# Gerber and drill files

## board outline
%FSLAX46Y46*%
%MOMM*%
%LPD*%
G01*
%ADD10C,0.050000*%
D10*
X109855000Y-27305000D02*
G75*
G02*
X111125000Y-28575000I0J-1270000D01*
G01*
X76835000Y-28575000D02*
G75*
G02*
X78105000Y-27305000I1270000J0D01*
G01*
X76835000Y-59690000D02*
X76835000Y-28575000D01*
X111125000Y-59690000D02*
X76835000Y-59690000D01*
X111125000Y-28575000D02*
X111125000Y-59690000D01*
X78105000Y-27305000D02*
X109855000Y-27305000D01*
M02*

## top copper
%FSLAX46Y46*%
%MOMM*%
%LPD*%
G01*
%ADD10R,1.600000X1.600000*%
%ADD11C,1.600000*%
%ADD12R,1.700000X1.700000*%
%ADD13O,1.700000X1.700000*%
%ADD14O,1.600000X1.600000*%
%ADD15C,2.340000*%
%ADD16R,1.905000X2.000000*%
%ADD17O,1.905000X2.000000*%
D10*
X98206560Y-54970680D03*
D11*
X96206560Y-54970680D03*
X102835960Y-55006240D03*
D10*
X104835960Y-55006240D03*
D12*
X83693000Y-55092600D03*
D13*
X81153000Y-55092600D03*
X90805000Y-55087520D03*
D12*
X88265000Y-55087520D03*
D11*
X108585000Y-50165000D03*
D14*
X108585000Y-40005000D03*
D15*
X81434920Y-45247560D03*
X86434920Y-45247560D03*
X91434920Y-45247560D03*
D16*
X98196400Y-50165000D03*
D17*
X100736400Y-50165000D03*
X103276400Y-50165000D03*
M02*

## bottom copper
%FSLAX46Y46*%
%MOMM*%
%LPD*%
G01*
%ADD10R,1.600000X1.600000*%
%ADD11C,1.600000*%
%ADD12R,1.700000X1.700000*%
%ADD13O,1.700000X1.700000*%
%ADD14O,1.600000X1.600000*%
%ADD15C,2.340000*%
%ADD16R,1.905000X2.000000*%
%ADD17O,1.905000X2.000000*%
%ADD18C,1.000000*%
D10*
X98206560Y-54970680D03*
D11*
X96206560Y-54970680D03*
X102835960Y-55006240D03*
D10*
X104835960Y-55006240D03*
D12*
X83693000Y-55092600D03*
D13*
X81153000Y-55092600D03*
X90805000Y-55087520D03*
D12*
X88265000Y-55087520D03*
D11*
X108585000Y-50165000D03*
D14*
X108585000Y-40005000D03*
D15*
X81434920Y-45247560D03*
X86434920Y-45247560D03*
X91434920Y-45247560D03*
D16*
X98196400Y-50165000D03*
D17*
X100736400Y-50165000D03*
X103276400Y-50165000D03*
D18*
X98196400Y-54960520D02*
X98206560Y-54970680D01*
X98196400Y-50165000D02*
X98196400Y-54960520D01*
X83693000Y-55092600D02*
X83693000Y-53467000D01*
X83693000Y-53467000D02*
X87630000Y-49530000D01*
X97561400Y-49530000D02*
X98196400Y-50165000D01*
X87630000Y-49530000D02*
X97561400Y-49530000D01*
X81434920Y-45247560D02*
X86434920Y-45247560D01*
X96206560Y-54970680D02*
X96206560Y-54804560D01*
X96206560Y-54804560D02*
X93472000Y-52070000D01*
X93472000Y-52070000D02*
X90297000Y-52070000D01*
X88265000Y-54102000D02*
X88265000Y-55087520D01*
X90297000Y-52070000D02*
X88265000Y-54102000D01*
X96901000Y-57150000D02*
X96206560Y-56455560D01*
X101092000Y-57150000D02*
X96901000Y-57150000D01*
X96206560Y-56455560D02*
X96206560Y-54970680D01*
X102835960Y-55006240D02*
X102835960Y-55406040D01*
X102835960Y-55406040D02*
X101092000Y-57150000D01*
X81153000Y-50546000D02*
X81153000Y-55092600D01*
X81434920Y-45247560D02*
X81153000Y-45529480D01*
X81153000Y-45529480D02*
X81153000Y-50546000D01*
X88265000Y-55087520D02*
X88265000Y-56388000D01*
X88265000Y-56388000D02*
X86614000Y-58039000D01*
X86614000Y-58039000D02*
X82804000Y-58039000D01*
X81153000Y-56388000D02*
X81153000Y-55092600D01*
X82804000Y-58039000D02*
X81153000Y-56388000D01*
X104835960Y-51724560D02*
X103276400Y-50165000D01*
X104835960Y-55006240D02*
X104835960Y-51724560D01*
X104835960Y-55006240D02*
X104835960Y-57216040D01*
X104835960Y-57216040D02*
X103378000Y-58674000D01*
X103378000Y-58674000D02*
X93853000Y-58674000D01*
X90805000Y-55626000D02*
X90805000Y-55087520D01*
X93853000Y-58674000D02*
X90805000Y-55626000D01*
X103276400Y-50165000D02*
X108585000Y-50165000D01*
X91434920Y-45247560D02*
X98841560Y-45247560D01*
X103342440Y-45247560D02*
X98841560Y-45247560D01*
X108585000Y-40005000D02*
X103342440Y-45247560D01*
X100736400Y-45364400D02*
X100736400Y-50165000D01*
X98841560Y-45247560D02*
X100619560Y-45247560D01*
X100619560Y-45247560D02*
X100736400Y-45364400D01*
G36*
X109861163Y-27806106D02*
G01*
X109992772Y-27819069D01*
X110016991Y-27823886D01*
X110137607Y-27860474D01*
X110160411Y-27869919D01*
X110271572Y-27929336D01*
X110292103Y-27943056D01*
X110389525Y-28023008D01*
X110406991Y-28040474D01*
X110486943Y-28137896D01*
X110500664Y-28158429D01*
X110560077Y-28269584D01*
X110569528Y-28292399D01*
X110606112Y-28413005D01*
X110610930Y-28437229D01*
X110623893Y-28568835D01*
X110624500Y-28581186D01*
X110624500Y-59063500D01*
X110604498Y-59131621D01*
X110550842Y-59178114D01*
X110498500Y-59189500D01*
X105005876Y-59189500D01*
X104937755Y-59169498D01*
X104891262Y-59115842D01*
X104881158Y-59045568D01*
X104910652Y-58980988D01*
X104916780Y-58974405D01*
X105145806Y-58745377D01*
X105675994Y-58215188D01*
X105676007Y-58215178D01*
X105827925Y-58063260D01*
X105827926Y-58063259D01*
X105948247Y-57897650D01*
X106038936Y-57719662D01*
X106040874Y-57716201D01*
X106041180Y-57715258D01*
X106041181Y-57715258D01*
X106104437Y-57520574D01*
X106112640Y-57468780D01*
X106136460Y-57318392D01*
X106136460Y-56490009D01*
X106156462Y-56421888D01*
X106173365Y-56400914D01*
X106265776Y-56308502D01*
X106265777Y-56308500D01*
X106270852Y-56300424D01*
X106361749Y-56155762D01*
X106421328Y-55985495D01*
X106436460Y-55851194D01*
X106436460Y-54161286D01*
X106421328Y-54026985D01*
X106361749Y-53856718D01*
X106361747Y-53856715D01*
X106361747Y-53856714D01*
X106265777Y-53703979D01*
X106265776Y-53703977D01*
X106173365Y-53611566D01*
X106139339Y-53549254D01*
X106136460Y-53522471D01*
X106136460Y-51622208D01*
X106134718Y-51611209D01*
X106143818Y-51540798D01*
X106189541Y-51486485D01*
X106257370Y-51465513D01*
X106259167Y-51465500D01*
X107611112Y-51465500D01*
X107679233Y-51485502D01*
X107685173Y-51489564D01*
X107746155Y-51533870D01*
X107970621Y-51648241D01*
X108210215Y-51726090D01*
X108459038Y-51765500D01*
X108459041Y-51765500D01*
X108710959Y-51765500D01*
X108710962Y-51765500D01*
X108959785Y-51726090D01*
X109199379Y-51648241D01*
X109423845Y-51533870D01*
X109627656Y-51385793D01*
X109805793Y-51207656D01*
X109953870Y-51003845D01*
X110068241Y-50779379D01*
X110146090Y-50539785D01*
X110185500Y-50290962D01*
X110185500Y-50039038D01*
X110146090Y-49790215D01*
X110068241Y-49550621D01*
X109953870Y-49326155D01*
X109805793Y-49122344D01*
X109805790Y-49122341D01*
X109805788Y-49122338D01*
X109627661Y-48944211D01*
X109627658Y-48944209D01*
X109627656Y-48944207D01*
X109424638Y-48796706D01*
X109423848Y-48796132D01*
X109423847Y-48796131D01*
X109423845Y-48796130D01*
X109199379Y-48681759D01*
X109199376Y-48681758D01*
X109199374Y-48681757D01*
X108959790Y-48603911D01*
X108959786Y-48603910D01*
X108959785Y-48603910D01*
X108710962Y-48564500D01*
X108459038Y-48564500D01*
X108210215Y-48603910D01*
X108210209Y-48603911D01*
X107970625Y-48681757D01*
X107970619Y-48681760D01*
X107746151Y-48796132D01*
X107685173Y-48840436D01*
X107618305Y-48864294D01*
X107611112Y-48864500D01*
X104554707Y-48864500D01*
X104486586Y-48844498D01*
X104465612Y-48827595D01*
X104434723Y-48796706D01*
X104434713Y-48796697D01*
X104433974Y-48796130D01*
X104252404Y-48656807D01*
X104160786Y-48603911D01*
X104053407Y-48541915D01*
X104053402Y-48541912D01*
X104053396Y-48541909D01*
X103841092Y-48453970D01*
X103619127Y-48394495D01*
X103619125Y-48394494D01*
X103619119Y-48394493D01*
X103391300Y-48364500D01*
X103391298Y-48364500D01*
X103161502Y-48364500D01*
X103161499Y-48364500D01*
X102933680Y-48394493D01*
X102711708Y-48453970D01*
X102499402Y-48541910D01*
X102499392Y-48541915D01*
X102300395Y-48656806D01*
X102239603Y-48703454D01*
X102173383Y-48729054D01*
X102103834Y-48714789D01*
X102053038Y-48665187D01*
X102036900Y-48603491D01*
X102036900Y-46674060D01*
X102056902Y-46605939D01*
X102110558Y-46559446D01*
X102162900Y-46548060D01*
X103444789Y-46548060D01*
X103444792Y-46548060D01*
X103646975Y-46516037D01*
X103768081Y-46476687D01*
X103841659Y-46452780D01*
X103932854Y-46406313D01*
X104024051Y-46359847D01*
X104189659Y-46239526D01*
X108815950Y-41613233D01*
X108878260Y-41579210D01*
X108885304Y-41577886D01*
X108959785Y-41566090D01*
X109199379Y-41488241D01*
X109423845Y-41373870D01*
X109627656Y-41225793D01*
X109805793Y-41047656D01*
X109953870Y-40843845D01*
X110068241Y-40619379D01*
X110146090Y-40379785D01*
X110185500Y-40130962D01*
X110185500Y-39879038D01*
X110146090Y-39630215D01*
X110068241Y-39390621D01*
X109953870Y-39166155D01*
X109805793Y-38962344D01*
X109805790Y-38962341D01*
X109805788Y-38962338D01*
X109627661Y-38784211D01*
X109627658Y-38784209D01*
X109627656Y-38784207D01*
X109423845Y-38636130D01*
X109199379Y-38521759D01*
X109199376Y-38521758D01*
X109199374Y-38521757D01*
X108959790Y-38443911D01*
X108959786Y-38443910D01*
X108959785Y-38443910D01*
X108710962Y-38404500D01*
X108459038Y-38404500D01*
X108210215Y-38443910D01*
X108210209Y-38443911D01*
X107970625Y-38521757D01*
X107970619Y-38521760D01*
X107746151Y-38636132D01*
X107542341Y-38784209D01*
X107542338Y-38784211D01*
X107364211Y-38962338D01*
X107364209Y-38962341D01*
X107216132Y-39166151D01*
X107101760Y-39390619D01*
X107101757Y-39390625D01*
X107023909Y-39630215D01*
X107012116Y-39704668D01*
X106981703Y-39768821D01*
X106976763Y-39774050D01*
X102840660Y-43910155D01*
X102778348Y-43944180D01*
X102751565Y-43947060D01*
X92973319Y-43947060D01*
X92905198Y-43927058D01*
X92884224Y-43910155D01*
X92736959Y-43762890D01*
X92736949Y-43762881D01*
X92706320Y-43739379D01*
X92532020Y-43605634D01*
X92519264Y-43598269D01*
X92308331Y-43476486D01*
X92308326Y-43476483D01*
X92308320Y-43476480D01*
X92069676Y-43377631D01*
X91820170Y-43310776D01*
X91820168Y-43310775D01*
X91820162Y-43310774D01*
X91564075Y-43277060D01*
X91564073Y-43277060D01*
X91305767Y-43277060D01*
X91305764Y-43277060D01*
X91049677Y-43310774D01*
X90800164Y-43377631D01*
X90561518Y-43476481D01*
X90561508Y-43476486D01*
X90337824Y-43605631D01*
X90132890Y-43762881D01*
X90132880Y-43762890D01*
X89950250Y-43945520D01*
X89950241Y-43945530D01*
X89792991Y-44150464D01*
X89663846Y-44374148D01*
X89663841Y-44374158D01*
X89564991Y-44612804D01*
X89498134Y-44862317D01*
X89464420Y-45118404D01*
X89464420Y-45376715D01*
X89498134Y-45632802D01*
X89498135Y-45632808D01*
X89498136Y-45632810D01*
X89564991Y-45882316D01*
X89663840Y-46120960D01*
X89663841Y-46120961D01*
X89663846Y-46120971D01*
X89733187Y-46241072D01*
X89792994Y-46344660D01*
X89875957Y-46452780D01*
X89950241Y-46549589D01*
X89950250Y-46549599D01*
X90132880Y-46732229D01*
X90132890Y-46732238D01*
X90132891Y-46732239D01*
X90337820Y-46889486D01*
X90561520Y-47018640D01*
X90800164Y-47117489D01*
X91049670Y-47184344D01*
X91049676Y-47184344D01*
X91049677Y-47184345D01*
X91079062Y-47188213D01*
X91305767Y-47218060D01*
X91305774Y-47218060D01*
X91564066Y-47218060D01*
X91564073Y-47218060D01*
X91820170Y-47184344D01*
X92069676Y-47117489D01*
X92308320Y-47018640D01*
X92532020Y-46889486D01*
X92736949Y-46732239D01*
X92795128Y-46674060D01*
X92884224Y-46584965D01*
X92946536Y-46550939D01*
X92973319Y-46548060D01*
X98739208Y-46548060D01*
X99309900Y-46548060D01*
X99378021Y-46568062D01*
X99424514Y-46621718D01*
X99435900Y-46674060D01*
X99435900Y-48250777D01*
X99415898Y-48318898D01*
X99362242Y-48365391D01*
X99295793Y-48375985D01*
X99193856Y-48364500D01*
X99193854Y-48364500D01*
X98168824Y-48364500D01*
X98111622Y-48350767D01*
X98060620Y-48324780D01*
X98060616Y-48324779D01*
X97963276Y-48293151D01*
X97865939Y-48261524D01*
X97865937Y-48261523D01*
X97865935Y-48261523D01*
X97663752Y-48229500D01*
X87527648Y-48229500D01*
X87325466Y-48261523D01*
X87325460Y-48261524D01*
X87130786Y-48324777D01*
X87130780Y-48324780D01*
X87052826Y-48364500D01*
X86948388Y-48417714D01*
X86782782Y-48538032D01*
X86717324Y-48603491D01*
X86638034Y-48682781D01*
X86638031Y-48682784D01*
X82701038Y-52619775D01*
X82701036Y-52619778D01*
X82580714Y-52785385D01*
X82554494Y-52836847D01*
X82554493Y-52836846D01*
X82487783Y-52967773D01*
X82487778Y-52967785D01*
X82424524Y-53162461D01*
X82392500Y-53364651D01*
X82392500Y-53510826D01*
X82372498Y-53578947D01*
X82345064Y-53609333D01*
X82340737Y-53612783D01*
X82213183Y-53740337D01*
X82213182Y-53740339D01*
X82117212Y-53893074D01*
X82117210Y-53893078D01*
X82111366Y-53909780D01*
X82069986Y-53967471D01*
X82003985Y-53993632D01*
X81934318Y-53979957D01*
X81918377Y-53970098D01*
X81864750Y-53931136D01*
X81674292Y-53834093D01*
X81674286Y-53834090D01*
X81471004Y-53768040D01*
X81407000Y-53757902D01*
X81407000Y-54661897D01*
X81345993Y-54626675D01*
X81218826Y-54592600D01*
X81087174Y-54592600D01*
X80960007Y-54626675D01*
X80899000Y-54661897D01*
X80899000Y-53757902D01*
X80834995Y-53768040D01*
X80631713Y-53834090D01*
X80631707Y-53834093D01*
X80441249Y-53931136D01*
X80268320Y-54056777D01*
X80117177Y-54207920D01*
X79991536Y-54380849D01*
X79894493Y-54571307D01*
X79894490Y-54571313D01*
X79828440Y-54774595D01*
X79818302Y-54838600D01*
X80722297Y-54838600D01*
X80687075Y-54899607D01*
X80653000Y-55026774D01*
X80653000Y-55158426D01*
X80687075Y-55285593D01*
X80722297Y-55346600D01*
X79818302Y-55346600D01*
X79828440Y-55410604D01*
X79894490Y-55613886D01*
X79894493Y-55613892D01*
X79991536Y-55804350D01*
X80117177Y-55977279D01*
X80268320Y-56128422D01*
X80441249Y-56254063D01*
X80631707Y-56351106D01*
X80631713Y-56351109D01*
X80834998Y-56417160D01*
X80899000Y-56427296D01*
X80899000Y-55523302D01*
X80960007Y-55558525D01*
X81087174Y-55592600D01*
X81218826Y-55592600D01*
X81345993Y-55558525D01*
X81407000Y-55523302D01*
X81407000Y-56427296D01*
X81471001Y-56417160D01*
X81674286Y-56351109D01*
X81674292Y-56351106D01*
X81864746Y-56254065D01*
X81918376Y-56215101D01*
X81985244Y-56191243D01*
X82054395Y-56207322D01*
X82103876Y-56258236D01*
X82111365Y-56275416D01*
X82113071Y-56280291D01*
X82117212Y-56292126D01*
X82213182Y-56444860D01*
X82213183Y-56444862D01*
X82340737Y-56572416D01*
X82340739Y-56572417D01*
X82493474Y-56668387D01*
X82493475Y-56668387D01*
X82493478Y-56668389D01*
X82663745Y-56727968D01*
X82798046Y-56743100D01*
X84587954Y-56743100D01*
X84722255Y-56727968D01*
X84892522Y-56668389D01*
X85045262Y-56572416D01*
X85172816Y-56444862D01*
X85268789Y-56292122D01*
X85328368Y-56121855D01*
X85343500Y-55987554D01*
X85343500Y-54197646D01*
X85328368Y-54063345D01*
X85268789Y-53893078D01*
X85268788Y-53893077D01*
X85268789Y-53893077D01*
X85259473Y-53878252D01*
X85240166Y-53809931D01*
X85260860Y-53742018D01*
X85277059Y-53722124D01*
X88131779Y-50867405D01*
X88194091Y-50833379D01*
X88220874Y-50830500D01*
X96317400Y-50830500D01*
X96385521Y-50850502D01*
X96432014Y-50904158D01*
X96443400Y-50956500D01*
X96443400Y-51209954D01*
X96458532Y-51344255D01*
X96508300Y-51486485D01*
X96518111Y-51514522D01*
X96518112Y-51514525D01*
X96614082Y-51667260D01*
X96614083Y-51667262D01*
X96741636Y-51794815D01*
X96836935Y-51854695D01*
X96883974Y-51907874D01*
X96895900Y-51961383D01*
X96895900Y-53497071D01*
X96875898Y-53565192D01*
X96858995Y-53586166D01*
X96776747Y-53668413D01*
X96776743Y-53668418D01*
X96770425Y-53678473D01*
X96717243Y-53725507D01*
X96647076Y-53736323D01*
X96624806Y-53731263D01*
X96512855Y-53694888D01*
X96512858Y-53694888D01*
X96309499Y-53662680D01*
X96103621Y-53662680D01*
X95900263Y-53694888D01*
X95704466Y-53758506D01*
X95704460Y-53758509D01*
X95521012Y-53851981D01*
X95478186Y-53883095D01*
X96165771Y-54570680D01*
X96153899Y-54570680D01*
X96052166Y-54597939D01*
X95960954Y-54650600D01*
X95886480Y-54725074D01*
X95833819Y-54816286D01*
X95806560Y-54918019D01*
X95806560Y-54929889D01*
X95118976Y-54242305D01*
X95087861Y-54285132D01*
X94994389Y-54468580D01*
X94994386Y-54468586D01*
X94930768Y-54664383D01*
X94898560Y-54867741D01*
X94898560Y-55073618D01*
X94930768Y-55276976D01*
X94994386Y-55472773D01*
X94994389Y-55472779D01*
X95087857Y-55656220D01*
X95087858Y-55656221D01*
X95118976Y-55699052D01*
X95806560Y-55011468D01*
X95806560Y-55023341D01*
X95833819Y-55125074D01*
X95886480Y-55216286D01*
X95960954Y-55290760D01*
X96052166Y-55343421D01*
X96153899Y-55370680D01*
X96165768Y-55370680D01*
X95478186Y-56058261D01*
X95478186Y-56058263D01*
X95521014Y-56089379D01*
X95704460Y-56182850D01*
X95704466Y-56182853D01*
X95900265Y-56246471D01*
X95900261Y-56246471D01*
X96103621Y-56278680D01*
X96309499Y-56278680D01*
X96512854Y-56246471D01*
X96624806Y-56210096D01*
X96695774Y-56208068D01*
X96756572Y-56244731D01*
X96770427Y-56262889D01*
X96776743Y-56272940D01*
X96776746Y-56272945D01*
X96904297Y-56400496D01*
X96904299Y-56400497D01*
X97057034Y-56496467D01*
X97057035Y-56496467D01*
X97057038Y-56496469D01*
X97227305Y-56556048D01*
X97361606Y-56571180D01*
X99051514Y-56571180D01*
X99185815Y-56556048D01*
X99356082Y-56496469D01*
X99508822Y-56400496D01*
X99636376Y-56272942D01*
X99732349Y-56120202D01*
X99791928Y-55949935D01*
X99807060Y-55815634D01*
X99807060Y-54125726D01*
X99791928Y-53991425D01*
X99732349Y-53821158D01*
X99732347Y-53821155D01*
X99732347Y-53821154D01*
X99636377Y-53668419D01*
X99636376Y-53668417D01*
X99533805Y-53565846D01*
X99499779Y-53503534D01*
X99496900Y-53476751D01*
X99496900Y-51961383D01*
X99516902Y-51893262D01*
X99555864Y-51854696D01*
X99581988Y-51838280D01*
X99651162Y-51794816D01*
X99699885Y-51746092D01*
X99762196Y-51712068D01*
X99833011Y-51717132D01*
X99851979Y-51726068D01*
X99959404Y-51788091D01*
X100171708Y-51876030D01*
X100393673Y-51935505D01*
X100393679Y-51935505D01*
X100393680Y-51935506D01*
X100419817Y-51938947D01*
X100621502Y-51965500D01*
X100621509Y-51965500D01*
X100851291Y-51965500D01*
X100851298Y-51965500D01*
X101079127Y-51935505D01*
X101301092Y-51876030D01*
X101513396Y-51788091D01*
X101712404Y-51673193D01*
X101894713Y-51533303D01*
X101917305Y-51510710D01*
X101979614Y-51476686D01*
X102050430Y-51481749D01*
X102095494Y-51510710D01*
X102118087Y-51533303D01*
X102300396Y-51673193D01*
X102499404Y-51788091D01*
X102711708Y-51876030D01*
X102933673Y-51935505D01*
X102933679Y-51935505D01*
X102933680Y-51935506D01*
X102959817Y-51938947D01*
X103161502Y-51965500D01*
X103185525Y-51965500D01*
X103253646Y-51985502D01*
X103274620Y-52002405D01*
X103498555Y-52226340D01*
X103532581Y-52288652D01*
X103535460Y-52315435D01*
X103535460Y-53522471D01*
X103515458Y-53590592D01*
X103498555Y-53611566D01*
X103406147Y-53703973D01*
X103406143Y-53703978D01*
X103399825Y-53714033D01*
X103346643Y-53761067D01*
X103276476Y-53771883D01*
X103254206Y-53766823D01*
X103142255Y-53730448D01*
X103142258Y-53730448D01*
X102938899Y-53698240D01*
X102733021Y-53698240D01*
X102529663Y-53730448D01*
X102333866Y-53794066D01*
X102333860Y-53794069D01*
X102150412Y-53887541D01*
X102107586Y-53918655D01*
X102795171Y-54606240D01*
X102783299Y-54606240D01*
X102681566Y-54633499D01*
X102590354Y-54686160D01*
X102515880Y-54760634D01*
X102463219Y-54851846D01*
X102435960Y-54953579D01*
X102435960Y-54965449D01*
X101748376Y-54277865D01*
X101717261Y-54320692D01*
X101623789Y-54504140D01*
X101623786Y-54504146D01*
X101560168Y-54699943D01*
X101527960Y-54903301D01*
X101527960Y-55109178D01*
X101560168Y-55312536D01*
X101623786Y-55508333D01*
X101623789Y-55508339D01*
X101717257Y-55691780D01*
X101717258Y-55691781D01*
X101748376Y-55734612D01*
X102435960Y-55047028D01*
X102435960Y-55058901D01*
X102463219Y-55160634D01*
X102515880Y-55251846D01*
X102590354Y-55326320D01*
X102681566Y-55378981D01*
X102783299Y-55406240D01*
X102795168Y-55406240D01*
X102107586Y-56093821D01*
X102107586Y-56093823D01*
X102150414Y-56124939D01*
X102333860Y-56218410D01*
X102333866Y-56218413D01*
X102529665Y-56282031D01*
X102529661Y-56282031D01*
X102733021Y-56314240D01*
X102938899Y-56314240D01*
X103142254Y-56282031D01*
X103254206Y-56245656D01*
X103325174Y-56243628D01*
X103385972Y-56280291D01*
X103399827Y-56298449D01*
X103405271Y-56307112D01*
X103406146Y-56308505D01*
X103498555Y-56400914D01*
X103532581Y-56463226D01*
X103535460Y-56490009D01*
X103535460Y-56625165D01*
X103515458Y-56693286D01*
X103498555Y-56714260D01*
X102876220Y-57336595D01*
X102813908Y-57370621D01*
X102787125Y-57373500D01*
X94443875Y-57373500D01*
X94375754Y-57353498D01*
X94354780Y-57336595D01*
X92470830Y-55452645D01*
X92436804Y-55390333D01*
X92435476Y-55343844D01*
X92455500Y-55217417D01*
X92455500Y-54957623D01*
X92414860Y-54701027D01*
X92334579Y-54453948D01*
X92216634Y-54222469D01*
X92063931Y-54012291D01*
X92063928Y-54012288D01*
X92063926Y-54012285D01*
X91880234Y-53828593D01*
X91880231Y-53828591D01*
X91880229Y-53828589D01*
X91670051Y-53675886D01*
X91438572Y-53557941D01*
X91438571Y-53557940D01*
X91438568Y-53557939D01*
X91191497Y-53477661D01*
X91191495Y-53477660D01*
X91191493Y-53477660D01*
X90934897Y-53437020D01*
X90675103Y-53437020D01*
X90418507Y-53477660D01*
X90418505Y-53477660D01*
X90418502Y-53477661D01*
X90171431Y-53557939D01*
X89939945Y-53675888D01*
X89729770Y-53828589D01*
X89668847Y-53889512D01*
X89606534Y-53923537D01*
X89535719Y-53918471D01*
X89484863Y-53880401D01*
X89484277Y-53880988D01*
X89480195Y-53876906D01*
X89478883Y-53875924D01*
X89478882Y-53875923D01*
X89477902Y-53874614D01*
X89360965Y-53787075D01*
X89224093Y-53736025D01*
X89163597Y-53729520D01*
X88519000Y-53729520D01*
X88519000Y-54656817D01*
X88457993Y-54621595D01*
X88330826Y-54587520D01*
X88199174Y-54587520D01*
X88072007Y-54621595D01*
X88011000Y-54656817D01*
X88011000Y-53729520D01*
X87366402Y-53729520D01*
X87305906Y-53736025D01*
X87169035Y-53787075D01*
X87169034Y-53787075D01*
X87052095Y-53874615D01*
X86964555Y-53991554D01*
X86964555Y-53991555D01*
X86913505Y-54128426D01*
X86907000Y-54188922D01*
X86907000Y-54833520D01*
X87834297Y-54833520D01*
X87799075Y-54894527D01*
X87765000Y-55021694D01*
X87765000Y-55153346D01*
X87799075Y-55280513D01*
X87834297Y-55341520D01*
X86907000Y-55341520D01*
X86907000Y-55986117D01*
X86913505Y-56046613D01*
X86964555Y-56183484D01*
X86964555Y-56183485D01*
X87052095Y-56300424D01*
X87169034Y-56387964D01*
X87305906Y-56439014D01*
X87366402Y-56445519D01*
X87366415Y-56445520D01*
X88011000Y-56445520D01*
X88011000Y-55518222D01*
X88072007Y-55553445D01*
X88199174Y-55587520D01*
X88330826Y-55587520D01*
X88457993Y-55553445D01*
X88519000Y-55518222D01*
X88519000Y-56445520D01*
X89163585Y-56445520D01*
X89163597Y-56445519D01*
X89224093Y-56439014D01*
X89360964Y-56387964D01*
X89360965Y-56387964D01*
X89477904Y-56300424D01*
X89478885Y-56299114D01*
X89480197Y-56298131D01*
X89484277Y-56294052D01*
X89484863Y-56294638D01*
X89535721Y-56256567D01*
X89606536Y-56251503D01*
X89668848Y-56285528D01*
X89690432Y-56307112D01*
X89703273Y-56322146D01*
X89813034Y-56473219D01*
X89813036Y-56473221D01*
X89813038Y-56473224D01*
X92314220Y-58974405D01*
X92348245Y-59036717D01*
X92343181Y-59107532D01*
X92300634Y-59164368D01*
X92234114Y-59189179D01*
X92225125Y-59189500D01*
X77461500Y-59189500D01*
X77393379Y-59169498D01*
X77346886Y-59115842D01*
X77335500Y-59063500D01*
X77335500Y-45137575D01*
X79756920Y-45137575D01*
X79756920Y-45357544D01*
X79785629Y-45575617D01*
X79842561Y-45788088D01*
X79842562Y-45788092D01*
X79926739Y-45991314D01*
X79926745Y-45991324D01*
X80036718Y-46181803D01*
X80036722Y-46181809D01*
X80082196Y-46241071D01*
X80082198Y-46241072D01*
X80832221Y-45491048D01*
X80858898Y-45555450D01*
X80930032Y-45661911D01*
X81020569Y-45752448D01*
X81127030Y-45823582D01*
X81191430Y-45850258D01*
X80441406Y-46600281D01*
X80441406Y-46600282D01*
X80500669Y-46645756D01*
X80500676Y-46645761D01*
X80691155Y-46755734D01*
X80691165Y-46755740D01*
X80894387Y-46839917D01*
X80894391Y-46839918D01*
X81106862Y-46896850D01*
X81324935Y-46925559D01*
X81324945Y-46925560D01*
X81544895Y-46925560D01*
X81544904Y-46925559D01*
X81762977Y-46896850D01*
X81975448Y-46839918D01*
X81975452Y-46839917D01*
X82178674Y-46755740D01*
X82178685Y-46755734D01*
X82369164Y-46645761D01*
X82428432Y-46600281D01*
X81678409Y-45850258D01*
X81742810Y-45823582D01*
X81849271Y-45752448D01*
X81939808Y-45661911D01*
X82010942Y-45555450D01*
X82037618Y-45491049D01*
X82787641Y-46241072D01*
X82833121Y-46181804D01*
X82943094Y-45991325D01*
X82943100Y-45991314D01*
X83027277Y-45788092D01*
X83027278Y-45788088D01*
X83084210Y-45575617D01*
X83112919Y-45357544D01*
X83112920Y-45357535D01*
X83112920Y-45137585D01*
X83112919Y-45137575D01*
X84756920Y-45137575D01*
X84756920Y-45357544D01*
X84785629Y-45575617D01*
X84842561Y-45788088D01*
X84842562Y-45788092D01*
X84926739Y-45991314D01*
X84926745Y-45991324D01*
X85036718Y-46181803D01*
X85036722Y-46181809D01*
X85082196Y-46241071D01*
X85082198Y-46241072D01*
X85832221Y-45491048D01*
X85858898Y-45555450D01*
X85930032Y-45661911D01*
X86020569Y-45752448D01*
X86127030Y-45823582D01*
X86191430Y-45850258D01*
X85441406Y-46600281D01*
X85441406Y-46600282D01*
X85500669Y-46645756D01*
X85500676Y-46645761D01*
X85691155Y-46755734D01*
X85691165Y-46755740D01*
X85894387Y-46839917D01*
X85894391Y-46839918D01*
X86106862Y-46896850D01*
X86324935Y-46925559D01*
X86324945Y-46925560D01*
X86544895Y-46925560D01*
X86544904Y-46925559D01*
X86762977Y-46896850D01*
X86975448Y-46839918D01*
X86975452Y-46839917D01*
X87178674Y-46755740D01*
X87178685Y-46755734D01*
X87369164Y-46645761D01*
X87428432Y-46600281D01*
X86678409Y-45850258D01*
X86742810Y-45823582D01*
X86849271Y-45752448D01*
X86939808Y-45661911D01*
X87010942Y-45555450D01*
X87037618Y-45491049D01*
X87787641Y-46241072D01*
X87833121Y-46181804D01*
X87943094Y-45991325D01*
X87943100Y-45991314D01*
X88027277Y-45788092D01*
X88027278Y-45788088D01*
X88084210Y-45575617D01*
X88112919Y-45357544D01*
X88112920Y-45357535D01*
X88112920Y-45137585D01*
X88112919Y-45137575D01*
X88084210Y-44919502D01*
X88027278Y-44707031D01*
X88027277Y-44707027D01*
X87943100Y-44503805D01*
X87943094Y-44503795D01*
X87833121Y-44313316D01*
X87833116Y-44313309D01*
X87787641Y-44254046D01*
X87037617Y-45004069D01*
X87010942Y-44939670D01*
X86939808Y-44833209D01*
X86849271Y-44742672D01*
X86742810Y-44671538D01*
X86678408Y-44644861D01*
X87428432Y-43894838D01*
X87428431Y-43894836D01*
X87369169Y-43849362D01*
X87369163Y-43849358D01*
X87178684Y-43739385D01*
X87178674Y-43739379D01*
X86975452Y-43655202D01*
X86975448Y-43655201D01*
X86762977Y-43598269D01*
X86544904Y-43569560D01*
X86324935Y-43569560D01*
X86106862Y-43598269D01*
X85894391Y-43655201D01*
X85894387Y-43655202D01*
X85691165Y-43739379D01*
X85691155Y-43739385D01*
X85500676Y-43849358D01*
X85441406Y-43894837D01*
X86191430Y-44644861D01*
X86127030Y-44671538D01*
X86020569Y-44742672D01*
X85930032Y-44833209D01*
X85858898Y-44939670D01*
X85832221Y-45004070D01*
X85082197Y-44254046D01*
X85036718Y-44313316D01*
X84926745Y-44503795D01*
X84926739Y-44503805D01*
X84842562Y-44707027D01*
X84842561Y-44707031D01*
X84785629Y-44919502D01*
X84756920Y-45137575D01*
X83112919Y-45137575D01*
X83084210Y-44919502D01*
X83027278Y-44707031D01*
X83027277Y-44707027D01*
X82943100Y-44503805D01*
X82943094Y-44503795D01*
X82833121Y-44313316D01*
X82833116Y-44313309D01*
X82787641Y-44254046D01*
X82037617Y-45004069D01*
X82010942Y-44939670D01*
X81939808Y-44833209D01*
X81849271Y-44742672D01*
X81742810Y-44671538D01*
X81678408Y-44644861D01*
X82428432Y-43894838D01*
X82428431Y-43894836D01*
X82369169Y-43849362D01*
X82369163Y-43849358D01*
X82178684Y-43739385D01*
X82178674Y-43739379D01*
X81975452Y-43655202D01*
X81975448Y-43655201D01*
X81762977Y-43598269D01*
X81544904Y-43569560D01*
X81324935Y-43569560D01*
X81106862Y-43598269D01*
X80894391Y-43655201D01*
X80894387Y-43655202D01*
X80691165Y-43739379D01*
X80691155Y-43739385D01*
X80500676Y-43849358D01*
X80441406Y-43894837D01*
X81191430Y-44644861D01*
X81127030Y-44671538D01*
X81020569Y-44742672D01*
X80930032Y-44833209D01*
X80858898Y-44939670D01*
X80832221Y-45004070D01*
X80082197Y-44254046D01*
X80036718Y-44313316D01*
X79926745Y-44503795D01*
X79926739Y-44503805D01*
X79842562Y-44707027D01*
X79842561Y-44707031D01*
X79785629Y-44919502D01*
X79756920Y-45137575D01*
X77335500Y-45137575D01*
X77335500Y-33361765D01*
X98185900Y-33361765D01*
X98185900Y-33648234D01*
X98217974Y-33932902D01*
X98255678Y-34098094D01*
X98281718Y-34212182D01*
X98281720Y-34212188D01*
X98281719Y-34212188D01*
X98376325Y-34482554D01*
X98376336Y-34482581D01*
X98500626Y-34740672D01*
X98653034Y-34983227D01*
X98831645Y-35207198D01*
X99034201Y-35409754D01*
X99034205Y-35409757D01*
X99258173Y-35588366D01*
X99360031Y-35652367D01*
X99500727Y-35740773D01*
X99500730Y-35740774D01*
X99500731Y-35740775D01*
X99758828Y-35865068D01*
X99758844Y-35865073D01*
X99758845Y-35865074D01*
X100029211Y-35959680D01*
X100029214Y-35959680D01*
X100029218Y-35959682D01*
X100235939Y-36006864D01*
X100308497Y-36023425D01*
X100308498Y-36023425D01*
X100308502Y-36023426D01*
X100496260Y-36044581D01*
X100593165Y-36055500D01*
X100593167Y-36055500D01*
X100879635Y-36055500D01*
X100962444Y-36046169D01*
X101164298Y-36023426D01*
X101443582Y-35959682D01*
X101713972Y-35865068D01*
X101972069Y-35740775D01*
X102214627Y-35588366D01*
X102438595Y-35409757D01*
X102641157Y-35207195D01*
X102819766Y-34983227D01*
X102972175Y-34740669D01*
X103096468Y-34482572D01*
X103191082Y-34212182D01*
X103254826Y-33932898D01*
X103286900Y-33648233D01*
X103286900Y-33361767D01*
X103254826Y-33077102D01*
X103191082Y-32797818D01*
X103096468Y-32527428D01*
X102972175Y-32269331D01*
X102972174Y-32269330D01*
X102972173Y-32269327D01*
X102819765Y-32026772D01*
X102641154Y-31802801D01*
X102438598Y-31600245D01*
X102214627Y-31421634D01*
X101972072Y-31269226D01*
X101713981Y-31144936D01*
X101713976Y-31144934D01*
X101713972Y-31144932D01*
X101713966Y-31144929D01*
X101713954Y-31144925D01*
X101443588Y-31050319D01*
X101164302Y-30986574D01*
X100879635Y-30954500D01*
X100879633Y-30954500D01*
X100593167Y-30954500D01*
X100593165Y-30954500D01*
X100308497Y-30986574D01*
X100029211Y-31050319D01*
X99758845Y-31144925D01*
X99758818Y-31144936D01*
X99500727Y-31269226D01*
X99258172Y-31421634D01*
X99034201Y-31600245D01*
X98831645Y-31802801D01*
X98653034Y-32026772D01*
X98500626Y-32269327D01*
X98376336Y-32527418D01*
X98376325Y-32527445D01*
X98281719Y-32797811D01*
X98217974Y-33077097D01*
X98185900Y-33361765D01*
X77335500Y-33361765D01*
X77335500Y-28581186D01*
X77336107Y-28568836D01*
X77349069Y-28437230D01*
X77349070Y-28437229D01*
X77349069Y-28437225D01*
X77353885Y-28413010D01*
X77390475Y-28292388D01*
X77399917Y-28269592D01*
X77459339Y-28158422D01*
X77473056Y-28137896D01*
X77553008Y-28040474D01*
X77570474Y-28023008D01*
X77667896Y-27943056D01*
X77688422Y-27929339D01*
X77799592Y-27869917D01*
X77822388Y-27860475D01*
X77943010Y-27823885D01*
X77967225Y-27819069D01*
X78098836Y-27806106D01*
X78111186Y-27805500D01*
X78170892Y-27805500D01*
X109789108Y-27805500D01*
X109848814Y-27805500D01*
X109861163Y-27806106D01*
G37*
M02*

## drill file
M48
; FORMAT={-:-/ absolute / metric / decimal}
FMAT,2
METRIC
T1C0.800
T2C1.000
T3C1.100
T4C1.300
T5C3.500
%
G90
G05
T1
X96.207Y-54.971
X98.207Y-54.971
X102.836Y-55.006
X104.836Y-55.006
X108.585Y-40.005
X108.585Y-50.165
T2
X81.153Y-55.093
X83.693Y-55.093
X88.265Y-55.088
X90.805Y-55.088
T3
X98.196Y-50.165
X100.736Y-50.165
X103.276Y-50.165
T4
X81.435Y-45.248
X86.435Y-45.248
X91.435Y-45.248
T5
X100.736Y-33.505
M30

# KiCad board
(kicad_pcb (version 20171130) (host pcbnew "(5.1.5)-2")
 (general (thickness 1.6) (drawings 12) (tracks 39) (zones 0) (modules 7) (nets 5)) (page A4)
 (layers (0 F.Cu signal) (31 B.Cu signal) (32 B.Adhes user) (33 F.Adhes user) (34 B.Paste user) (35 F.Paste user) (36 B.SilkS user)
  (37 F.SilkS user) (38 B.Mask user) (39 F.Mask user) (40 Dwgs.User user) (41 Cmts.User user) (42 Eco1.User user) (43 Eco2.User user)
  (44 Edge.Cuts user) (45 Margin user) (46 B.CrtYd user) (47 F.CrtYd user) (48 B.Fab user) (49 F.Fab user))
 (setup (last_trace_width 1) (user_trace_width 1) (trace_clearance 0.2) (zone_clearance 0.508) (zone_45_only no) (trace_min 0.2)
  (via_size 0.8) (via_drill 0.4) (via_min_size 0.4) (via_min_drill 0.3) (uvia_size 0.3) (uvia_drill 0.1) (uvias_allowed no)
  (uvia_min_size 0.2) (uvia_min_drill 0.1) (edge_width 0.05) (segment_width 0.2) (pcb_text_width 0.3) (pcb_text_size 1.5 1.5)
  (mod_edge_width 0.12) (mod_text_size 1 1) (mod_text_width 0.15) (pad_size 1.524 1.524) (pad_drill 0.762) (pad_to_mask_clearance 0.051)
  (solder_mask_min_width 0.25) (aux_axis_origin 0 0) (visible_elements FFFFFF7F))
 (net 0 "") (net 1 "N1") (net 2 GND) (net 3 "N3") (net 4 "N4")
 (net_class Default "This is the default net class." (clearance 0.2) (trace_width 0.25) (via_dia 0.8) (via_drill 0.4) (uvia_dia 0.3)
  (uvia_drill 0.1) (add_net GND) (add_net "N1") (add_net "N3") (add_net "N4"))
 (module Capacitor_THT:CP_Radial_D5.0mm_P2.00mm (layer F.Cu) (at 98.20656 54.97068 180)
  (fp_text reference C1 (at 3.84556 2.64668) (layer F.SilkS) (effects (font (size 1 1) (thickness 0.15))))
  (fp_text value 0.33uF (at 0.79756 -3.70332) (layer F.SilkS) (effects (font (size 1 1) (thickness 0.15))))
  (pad 1 thru_hole rect (at 0 0 180) (size 1.6 1.6) (drill 0.8) (layers *.Cu *.Mask) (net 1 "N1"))
  (pad 2 thru_hole circle (at 2 0 180) (size 1.6 1.6) (drill 0.8) (layers *.Cu *.Mask) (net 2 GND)))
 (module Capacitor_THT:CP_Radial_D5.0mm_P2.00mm (layer F.Cu) (at 104.83596 55.00624 180)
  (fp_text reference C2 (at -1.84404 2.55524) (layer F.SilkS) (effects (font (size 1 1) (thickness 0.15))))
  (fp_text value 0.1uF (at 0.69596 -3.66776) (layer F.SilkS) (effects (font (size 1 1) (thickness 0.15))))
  (pad 2 thru_hole circle (at 2 0 180) (size 1.6 1.6) (drill 0.8) (layers *.Cu *.Mask) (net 2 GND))
  (pad 1 thru_hole rect (at 0 0 180) (size 1.6 1.6) (drill 0.8) (layers *.Cu *.Mask) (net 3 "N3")))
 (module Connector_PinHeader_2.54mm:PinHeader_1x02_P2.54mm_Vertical (layer F.Cu) (at 83.693 55.0926 270)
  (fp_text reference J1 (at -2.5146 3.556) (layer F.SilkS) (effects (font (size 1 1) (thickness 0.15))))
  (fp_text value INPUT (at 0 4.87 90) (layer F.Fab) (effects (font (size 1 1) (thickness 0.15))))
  (pad 1 thru_hole rect (at 0 0 270) (size 1.7 1.7) (drill 1) (layers *.Cu *.Mask) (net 1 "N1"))
  (pad 2 thru_hole oval (at 0 2.54 270) (size 1.7 1.7) (drill 1) (layers *.Cu *.Mask) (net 2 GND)))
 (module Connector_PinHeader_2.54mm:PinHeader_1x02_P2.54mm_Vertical (layer F.Cu) (at 88.265 55.08752 90)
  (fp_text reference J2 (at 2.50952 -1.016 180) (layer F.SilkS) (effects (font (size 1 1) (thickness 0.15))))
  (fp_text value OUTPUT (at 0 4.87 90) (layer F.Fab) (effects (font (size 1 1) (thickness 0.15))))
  (pad 2 thru_hole oval (at 0 2.54 90) (size 1.7 1.7) (drill 1) (layers *.Cu *.Mask) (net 3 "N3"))
  (pad 1 thru_hole rect (at 0 0 90) (size 1.7 1.7) (drill 1) (layers *.Cu *.Mask) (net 2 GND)))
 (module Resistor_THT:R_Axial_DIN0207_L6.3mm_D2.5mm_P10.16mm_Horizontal (layer F.Cu) (at 108.585 50.165 90)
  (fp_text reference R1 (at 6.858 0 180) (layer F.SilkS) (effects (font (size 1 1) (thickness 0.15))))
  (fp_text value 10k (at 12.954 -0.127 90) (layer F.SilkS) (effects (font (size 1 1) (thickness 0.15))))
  (pad 1 thru_hole circle (at 0 0 90) (size 1.6 1.6) (drill 0.8) (layers *.Cu *.Mask) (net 3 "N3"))
  (pad 2 thru_hole oval (at 10.16 0 90) (size 1.6 1.6) (drill 0.8) (layers *.Cu *.Mask) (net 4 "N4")))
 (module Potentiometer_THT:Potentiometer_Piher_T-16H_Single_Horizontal (layer F.Cu) (at 91.43492 45.24756 90)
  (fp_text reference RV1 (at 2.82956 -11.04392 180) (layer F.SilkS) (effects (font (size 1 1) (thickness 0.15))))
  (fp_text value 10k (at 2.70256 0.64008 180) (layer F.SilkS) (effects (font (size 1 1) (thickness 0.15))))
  (pad 3 thru_hole circle (at 0 -10 90) (size 2.34 2.34) (drill 1.3) (layers *.Cu *.Mask) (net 2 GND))
  (pad 2 thru_hole circle (at 0 -5 90) (size 2.34 2.34) (drill 1.3) (layers *.Cu *.Mask) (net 2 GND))
  (pad 1 thru_hole circle (at 0 0 90) (size 2.34 2.34) (drill 1.3) (layers *.Cu *.Mask) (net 4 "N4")))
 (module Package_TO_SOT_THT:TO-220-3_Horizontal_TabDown (layer F.Cu) (at 98.1964 50.165)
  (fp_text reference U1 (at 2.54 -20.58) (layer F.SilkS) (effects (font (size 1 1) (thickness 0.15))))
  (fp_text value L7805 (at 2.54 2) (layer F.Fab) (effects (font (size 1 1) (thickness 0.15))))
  (pad "" np_thru_hole oval (at 2.54 -16.66) (size 3.5 3.5) (drill 3.5) (layers *.Cu *.Mask))
  (pad 1 thru_hole rect (at 0 0) (size 1.905 2) (drill 1.1) (layers *.Cu *.Mask) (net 1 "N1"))
  (pad 2 thru_hole oval (at 2.54 0) (size 1.905 2) (drill 1.1) (layers *.Cu *.Mask) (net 4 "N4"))
  (pad 3 thru_hole oval (at 5.08 0) (size 1.905 2) (drill 1.1) (layers *.Cu *.Mask) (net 3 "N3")))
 (gr_arc (start 109.855 28.575) (end 111.125 28.575) (angle -90) (layer Edge.Cuts) (width 0.05))
 (gr_arc (start 78.105 28.575) (end 78.105 27.305) (angle -90) (layer Edge.Cuts) (width 0.05))
 (gr_line (start 76.835 59.69) (end 76.835 28.575) (layer Edge.Cuts) (width 0.05))
 (gr_line (start 111.125 59.69) (end 76.835 59.69) (layer Edge.Cuts) (width 0.05))
 (gr_line (start 111.125 28.575) (end 111.125 59.69) (layer Edge.Cuts) (width 0.05))
 (gr_line (start 78.105 27.305) (end 109.855 27.305) (layer Edge.Cuts) (width 0.05))
 (segment (start 98.1964 54.96052) (end 98.20656 54.97068) (width 1) (layer B.Cu) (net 1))
 (segment (start 98.1964 50.165) (end 98.1964 54.96052) (width 1) (layer B.Cu) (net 1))
 (segment (start 83.693 55.0926) (end 83.693 53.467) (width 1) (layer B.Cu) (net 1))
 (segment (start 83.693 53.467) (end 87.63 49.53) (width 1) (layer B.Cu) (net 1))
 (segment (start 97.5614 49.53) (end 98.1964 50.165) (width 1) (layer B.Cu) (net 1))
 (segment (start 87.63 49.53) (end 97.5614 49.53) (width 1) (layer B.Cu) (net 1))
 (segment (start 81.43492 45.24756) (end 86.43492 45.24756) (width 1) (layer B.Cu) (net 2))
 (segment (start 96.20656 54.97068) (end 96.20656 54.80456) (width 1) (layer B.Cu) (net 2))
 (segment (start 96.20656 54.80456) (end 93.472 52.07) (width 1) (layer B.Cu) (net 2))
 (segment (start 93.472 52.07) (end 90.297 52.07) (width 1) (layer B.Cu) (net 2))
 (segment (start 88.265 54.102) (end 88.265 55.08752) (width 1) (layer B.Cu) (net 2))
 (segment (start 90.297 52.07) (end 88.265 54.102) (width 1) (layer B.Cu) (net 2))
 (segment (start 96.901 57.15) (end 96.20656 56.45556) (width 1) (layer B.Cu) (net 2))
 (segment (start 101.092 57.15) (end 96.901 57.15) (width 1) (layer B.Cu) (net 2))
 (segment (start 96.20656 56.45556) (end 96.20656 54.97068) (width 1) (layer B.Cu) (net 2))
 (segment (start 102.83596 55.00624) (end 102.83596 55.40604) (width 1) (layer B.Cu) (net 2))
 (segment (start 102.83596 55.40604) (end 101.092 57.15) (width 1) (layer B.Cu) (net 2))
 (segment (start 81.153 50.546) (end 81.153 55.0926) (width 1) (layer B.Cu) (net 2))
 (segment (start 81.43492 45.24756) (end 81.153 45.52948) (width 1) (layer B.Cu) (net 2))
 (segment (start 81.153 45.52948) (end 81.153 50.546) (width 1) (layer B.Cu) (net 2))
 (segment (start 88.265 55.08752) (end 88.265 56.388) (width 1) (layer B.Cu) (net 2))
 (segment (start 88.265 56.388) (end 86.614 58.039) (width 1) (layer B.Cu) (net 2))
 (segment (start 86.614 58.039) (end 82.804 58.039) (width 1) (layer B.Cu) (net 2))
 (segment (start 81.153 56.388) (end 81.153 55.0926) (width 1) (layer B.Cu) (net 2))
 (segment (start 82.804 58.039) (end 81.153 56.388) (width 1) (layer B.Cu) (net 2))
 (segment (start 104.83596 51.72456) (end 103.2764 50.165) (width 1) (layer B.Cu) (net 3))
 (segment (start 104.83596 55.00624) (end 104.83596 51.72456) (width 1) (layer B.Cu) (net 3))
 (segment (start 104.83596 55.00624) (end 104.83596 57.21604) (width 1) (layer B.Cu) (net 3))
 (segment (start 104.83596 57.21604) (end 103.378 58.674) (width 1) (layer B.Cu) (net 3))
 (segment (start 103.378 58.674) (end 93.853 58.674) (width 1) (layer B.Cu) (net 3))
 (segment (start 90.805 55.626) (end 90.805 55.08752) (width 1) (layer B.Cu) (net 3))
 (segment (start 93.853 58.674) (end 90.805 55.626) (width 1) (layer B.Cu) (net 3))
 (segment (start 103.2764 50.165) (end 108.585 50.165) (width 1) (layer B.Cu) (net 3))
 (segment (start 91.43492 45.24756) (end 98.84156 45.24756) (width 1) (layer B.Cu) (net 4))
 (segment (start 103.34244 45.24756) (end 98.84156 45.24756) (width 1) (layer B.Cu) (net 4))
 (segment (start 108.585 40.005) (end 103.34244 45.24756) (width 1) (layer B.Cu) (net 4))
 (segment (start 100.7364 45.3644) (end 100.7364 50.165) (width 1) (layer B.Cu) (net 4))
 (segment (start 98.84156 45.24756) (end 100.61956 45.24756) (width 1) (layer B.Cu) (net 4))
 (segment (start 100.61956 45.24756) (end 100.7364 45.3644) (width 1) (layer B.Cu) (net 4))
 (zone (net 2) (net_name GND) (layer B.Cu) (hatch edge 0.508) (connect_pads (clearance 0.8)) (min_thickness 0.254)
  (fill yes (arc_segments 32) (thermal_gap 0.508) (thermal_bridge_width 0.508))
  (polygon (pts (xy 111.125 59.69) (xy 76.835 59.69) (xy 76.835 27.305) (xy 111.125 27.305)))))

